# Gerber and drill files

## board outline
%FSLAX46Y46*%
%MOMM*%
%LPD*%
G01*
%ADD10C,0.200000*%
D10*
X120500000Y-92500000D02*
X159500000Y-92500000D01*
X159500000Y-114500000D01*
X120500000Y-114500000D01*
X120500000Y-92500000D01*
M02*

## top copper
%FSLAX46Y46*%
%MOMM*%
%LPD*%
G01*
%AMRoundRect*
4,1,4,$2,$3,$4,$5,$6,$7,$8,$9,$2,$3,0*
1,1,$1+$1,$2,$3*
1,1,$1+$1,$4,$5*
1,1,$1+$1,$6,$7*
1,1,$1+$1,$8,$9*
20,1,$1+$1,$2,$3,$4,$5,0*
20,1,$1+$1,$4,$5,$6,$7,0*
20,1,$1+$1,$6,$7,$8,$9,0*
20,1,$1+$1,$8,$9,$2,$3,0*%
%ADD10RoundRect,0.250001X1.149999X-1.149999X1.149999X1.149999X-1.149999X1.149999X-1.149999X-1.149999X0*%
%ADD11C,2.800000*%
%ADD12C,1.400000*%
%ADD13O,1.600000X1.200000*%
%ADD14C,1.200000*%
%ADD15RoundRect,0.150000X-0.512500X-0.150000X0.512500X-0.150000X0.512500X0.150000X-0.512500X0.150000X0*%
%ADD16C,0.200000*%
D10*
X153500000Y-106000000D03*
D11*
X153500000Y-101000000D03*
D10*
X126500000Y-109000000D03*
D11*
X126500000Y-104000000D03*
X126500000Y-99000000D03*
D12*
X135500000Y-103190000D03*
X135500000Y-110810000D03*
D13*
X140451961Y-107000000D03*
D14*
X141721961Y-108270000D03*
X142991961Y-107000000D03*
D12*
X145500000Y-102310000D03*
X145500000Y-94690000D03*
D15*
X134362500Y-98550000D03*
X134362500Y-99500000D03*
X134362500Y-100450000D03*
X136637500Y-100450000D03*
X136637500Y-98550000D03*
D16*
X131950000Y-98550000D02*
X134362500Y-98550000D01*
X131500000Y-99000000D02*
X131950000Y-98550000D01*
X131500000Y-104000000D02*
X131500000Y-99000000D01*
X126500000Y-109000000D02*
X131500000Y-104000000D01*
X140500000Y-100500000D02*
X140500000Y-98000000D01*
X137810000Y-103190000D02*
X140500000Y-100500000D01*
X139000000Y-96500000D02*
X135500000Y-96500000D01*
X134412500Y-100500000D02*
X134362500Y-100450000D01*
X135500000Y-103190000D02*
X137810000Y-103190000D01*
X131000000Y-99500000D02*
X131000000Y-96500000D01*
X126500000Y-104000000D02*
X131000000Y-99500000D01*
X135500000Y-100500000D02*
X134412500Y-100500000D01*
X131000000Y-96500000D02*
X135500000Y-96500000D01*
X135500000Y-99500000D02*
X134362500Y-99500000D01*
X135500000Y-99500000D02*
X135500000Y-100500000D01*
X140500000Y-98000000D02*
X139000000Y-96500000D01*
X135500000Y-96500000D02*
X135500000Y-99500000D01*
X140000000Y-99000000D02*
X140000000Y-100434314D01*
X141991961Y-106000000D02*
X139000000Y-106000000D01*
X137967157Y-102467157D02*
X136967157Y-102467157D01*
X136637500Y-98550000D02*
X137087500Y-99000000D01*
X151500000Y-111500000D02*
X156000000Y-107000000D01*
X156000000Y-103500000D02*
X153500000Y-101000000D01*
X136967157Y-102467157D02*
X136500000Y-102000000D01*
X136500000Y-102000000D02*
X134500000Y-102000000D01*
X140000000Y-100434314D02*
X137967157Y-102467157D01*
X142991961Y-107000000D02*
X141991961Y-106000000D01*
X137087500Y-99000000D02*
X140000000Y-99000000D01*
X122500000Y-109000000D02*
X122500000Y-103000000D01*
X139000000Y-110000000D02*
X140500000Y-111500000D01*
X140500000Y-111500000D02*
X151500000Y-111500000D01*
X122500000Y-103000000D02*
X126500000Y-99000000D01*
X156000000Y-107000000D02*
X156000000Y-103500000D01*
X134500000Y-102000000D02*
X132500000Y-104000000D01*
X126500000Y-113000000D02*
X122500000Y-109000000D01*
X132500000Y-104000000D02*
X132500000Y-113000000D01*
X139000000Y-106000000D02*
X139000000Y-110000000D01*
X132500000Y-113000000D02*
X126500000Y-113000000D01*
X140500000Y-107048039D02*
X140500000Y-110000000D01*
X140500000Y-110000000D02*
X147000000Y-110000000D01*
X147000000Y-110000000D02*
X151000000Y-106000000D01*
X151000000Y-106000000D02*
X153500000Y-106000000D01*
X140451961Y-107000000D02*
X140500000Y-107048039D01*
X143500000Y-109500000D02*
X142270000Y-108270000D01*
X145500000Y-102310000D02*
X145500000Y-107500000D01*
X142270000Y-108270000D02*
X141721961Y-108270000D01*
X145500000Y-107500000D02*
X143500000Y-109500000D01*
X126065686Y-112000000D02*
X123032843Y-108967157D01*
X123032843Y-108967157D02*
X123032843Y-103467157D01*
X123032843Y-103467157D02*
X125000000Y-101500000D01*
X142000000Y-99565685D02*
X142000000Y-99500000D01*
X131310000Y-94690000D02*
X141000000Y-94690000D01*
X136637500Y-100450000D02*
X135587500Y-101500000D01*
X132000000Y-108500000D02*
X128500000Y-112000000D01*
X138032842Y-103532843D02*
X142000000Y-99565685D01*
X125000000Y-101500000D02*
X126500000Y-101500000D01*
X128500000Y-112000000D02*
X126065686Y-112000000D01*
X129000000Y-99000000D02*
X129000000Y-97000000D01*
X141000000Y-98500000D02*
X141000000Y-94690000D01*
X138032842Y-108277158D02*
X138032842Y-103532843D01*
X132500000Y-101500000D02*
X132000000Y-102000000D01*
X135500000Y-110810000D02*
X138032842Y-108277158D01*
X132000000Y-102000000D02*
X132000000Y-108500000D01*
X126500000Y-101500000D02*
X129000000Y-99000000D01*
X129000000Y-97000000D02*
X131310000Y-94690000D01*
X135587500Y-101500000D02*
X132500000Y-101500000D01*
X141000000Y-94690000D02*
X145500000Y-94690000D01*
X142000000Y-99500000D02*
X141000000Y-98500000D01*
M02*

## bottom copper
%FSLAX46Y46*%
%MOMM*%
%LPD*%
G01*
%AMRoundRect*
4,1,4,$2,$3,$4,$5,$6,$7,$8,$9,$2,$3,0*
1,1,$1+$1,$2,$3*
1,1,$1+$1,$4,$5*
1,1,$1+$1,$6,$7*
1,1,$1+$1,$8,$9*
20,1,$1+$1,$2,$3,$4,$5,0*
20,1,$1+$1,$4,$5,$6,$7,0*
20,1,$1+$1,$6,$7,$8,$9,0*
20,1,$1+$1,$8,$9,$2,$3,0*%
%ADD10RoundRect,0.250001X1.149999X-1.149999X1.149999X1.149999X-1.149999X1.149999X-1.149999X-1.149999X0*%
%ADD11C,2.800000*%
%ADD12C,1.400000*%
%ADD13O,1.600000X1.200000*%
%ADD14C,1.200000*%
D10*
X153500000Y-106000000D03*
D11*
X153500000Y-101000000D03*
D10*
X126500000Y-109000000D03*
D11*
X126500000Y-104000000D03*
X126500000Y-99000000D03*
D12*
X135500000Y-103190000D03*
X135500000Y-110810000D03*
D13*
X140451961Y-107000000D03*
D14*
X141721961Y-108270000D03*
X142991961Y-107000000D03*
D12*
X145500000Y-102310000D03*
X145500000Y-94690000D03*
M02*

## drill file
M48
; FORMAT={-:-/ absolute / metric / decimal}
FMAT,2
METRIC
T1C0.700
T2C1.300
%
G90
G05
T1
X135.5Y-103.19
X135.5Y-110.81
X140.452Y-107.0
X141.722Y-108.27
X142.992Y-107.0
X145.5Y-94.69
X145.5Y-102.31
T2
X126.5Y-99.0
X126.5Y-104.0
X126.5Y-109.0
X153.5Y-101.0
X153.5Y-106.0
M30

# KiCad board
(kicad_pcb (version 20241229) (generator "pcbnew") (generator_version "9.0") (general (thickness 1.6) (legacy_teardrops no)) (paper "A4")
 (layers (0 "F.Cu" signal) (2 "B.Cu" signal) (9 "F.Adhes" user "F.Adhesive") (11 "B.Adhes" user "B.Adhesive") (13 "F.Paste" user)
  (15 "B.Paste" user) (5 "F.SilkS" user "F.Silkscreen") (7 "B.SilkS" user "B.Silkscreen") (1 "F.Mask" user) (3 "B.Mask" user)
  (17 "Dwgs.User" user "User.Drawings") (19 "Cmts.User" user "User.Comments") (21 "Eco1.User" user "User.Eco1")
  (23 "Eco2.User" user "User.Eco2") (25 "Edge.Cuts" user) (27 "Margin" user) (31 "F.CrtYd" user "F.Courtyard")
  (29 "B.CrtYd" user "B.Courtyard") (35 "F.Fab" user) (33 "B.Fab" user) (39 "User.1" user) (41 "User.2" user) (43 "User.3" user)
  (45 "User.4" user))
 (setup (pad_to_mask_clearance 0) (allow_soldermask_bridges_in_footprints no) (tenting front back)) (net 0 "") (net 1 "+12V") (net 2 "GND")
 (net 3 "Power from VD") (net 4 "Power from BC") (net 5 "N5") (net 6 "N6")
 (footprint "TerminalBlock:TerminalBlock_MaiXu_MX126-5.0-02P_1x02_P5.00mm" (layer "F.Cu") (at 153.5 106 90)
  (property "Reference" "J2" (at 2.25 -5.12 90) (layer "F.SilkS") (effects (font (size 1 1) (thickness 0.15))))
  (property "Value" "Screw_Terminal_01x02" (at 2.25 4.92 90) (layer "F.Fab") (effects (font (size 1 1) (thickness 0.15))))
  (pad "1" thru_hole roundrect (at 0 0 90) (size 2.8 2.8) (drill 1.3) (layers "*.Cu" "*.Mask") (remove_unused_layers no)
   (roundrect_rratio 0.089286) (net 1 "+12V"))
  (pad "2" thru_hole circle (at 5 0 90) (size 2.8 2.8) (drill 1.3) (layers "*.Cu" "*.Mask") (remove_unused_layers no) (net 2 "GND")))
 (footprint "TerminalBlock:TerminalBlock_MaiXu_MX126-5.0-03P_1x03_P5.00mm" (layer "F.Cu") (at 126.5 109 90)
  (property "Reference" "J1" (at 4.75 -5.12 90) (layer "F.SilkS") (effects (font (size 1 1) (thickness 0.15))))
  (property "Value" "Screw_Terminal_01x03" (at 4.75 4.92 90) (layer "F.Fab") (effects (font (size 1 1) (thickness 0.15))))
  (pad "1" thru_hole roundrect (at 0 0 90) (size 2.8 2.8) (drill 1.3) (layers "*.Cu" "*.Mask") (remove_unused_layers no)
   (roundrect_rratio 0.089286) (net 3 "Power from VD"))
  (pad "2" thru_hole circle (at 5 0 90) (size 2.8 2.8) (drill 1.3) (layers "*.Cu" "*.Mask") (remove_unused_layers no)
   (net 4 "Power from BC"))
  (pad "3" thru_hole circle (at 10 0 90) (size 2.8 2.8) (drill 1.3) (layers "*.Cu" "*.Mask") (remove_unused_layers no) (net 2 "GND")))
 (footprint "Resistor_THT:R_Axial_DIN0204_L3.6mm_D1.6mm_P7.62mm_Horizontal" (layer "F.Cu") (at 135.5 103.19 -90)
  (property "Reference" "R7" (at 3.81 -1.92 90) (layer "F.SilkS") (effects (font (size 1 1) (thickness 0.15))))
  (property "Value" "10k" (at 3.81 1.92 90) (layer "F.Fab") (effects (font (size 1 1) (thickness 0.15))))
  (pad "1" thru_hole circle (at 0 0 270) (size 1.4 1.4) (drill 0.7) (layers "*.Cu" "*.Mask") (remove_unused_layers no)
   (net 4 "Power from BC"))
  (pad "2" thru_hole circle (at 7.62 0 270) (size 1.4 1.4) (drill 0.7) (layers "*.Cu" "*.Mask") (remove_unused_layers no) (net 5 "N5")))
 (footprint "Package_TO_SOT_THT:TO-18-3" (layer "F.Cu") (at 140.451961 107)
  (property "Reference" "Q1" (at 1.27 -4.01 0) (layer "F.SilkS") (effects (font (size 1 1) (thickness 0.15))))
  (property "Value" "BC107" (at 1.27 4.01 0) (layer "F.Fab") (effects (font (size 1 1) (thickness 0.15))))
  (pad "1" thru_hole oval (at 0 0) (size 1.6 1.2) (drill 0.7) (layers "*.Cu" "*.Mask") (remove_unused_layers no) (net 1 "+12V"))
  (pad "2" thru_hole circle (at 1.27 1.27) (size 1.2 1.2) (drill 0.7) (layers "*.Cu" "*.Mask") (remove_unused_layers no) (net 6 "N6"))
  (pad "3" thru_hole circle (at 2.54 0) (size 1.2 1.2) (drill 0.7) (layers "*.Cu" "*.Mask") (remove_unused_layers no) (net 2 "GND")))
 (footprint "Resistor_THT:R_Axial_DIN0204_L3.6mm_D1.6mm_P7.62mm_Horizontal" (layer "F.Cu") (at 145.5 102.31 90)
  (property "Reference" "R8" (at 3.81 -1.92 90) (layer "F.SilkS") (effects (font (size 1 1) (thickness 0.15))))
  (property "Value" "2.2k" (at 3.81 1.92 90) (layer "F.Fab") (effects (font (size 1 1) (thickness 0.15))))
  (pad "1" thru_hole circle (at 0 0 90) (size 1.4 1.4) (drill 0.7) (layers "*.Cu" "*.Mask") (remove_unused_layers no) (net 6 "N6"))
  (pad "2" thru_hole circle (at 7.62 0 90) (size 1.4 1.4) (drill 0.7) (layers "*.Cu" "*.Mask") (remove_unused_layers no) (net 5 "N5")))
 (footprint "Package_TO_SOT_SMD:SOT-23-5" (layer "F.Cu") (at 135.5 99.5)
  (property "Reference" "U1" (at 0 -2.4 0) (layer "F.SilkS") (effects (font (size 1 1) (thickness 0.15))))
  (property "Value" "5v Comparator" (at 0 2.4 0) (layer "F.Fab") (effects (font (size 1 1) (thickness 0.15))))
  (pad "1" smd roundrect (at -1.1375 -0.95) (size 1.325 0.6) (layers "F.Cu" "F.Mask" "F.Paste") (roundrect_rratio 0.25)
   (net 3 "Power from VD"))
  (pad "2" smd roundrect (at -1.1375 0) (size 1.325 0.6) (layers "F.Cu" "F.Mask" "F.Paste") (roundrect_rratio 0.25) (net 4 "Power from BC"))
  (pad "3" smd roundrect (at -1.1375 0.95) (size 1.325 0.6) (layers "F.Cu" "F.Mask" "F.Paste") (roundrect_rratio 0.25)
   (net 4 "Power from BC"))
  (pad "4" smd roundrect (at 1.1375 0.95) (size 1.325 0.6) (layers "F.Cu" "F.Mask" "F.Paste") (roundrect_rratio 0.25) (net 5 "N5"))
  (pad "5" smd roundrect (at 1.1375 -0.95) (size 1.325 0.6) (layers "F.Cu" "F.Mask" "F.Paste") (roundrect_rratio 0.25) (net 2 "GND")))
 (gr_rect (start 120.5 92.5) (end 159.5 114.5) (stroke (width 0.2) (type solid)) (fill no) (layer "Edge.Cuts"))
 (segment (start 131.95 98.55) (end 134.3625 98.55) (width 0.2) (layer "F.Cu") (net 3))
 (segment (start 131.5 99) (end 131.95 98.55) (width 0.2) (layer "F.Cu") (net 3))
 (segment (start 131.5 104) (end 131.5 99) (width 0.2) (layer "F.Cu") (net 3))
 (segment (start 126.5 109) (end 131.5 104) (width 0.2) (layer "F.Cu") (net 3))
 (segment (start 140.5 100.5) (end 140.5 98) (width 0.2) (layer "F.Cu") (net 4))
 (segment (start 137.81 103.19) (end 140.5 100.5) (width 0.2) (layer "F.Cu") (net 4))
 (segment (start 139 96.5) (end 135.5 96.5) (width 0.2) (layer "F.Cu") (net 4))
 (segment (start 134.4125 100.5) (end 134.3625 100.45) (width 0.2) (layer "F.Cu") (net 4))
 (segment (start 135.5 103.19) (end 137.81 103.19) (width 0.2) (layer "F.Cu") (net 4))
 (segment (start 131 99.5) (end 131 96.5) (width 0.2) (layer "F.Cu") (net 4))
 (segment (start 126.5 104) (end 131 99.5) (width 0.2) (layer "F.Cu") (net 4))
 (segment (start 135.5 100.5) (end 134.4125 100.5) (width 0.2) (layer "F.Cu") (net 4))
 (segment (start 131 96.5) (end 135.5 96.5) (width 0.2) (layer "F.Cu") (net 4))
 (segment (start 135.5 99.5) (end 134.3625 99.5) (width 0.2) (layer "F.Cu") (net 4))
 (segment (start 135.5 99.5) (end 135.5 100.5) (width 0.2) (layer "F.Cu") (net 4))
 (segment (start 140.5 98) (end 139 96.5) (width 0.2) (layer "F.Cu") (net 4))
 (segment (start 135.5 96.5) (end 135.5 99.5) (width 0.2) (layer "F.Cu") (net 4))
 (segment (start 140 99) (end 140 100.434314) (width 0.2) (layer "F.Cu") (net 2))
 (segment (start 141.991961 106) (end 139 106) (width 0.2) (layer "F.Cu") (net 2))
 (segment (start 137.967157 102.467157) (end 136.967157 102.467157) (width 0.2) (layer "F.Cu") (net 2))
 (segment (start 136.6375 98.55) (end 137.0875 99) (width 0.2) (layer "F.Cu") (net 2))
 (segment (start 151.5 111.5) (end 156 107) (width 0.2) (layer "F.Cu") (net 2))
 (segment (start 156 103.5) (end 153.5 101) (width 0.2) (layer "F.Cu") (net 2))
 (segment (start 136.967157 102.467157) (end 136.5 102) (width 0.2) (layer "F.Cu") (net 2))
 (segment (start 136.5 102) (end 134.5 102) (width 0.2) (layer "F.Cu") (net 2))
 (segment (start 140 100.434314) (end 137.967157 102.467157) (width 0.2) (layer "F.Cu") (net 2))
 (segment (start 142.991961 107) (end 141.991961 106) (width 0.2) (layer "F.Cu") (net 2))
 (segment (start 137.0875 99) (end 140 99) (width 0.2) (layer "F.Cu") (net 2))
 (segment (start 122.5 109) (end 122.5 103) (width 0.2) (layer "F.Cu") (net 2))
 (segment (start 139 110) (end 140.5 111.5) (width 0.2) (layer "F.Cu") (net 2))
 (segment (start 140.5 111.5) (end 151.5 111.5) (width 0.2) (layer "F.Cu") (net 2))
 (segment (start 122.5 103) (end 126.5 99) (width 0.2) (layer "F.Cu") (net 2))
 (segment (start 156 107) (end 156 103.5) (width 0.2) (layer "F.Cu") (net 2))
 (segment (start 134.5 102) (end 132.5 104) (width 0.2) (layer "F.Cu") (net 2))
 (segment (start 126.5 113) (end 122.5 109) (width 0.2) (layer "F.Cu") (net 2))
 (segment (start 132.5 104) (end 132.5 113) (width 0.2) (layer "F.Cu") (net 2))
 (segment (start 139 106) (end 139 110) (width 0.2) (layer "F.Cu") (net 2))
 (segment (start 132.5 113) (end 126.5 113) (width 0.2) (layer "F.Cu") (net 2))
 (segment (start 140.5 107.048039) (end 140.5 110) (width 0.2) (layer "F.Cu") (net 1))
 (segment (start 140.5 110) (end 147 110) (width 0.2) (layer "F.Cu") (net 1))
 (segment (start 147 110) (end 151 106) (width 0.2) (layer "F.Cu") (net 1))
 (segment (start 151 106) (end 153.5 106) (width 0.2) (layer "F.Cu") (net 1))
 (segment (start 140.451961 107) (end 140.5 107.048039) (width 0.2) (layer "F.Cu") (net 1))
 (segment (start 143.5 109.5) (end 142.27 108.27) (width 0.2) (layer "F.Cu") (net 6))
 (segment (start 145.5 102.31) (end 145.5 107.5) (width 0.2) (layer "F.Cu") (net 6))
 (segment (start 142.27 108.27) (end 141.721961 108.27) (width 0.2) (layer "F.Cu") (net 6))
 (segment (start 145.5 107.5) (end 143.5 109.5) (width 0.2) (layer "F.Cu") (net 6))
 (segment (start 126.065686 112) (end 123.032843 108.967157) (width 0.2) (layer "F.Cu") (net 5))
 (segment (start 123.032843 108.967157) (end 123.032843 103.467157) (width 0.2) (layer "F.Cu") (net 5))
 (segment (start 123.032843 103.467157) (end 125 101.5) (width 0.2) (layer "F.Cu") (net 5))
 (segment (start 142 99.565685) (end 142 99.5) (width 0.2) (layer "F.Cu") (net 5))
 (segment (start 131.31 94.69) (end 141 94.69) (width 0.2) (layer "F.Cu") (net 5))
 (segment (start 136.6375 100.45) (end 135.5875 101.5) (width 0.2) (layer "F.Cu") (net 5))
 (segment (start 132 108.5) (end 128.5 112) (width 0.2) (layer "F.Cu") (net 5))
 (segment (start 138.032842 103.532843) (end 142 99.565685) (width 0.2) (layer "F.Cu") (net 5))
 (segment (start 125 101.5) (end 126.5 101.5) (width 0.2) (layer "F.Cu") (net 5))
 (segment (start 128.5 112) (end 126.065686 112) (width 0.2) (layer "F.Cu") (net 5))
 (segment (start 129 99) (end 129 97) (width 0.2) (layer "F.Cu") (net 5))
 (segment (start 141 98.5) (end 141 94.69) (width 0.2) (layer "F.Cu") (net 5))
 (segment (start 138.032842 108.277158) (end 138.032842 103.532843) (width 0.2) (layer "F.Cu") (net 5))
 (segment (start 132.5 101.5) (end 132 102) (width 0.2) (layer "F.Cu") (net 5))
 (segment (start 135.5 110.81) (end 138.032842 108.277158) (width 0.2) (layer "F.Cu") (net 5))
 (segment (start 132 102) (end 132 108.5) (width 0.2) (layer "F.Cu") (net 5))
 (segment (start 126.5 101.5) (end 129 99) (width 0.2) (layer "F.Cu") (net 5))
 (segment (start 129 97) (end 131.31 94.69) (width 0.2) (layer "F.Cu") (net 5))
 (segment (start 135.5875 101.5) (end 132.5 101.5) (width 0.2) (layer "F.Cu") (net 5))
 (segment (start 141 94.69) (end 145.5 94.69) (width 0.2) (layer "F.Cu") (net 5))
 (segment (start 142 99.5) (end 141 98.5) (width 0.2) (layer "F.Cu") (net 5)))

